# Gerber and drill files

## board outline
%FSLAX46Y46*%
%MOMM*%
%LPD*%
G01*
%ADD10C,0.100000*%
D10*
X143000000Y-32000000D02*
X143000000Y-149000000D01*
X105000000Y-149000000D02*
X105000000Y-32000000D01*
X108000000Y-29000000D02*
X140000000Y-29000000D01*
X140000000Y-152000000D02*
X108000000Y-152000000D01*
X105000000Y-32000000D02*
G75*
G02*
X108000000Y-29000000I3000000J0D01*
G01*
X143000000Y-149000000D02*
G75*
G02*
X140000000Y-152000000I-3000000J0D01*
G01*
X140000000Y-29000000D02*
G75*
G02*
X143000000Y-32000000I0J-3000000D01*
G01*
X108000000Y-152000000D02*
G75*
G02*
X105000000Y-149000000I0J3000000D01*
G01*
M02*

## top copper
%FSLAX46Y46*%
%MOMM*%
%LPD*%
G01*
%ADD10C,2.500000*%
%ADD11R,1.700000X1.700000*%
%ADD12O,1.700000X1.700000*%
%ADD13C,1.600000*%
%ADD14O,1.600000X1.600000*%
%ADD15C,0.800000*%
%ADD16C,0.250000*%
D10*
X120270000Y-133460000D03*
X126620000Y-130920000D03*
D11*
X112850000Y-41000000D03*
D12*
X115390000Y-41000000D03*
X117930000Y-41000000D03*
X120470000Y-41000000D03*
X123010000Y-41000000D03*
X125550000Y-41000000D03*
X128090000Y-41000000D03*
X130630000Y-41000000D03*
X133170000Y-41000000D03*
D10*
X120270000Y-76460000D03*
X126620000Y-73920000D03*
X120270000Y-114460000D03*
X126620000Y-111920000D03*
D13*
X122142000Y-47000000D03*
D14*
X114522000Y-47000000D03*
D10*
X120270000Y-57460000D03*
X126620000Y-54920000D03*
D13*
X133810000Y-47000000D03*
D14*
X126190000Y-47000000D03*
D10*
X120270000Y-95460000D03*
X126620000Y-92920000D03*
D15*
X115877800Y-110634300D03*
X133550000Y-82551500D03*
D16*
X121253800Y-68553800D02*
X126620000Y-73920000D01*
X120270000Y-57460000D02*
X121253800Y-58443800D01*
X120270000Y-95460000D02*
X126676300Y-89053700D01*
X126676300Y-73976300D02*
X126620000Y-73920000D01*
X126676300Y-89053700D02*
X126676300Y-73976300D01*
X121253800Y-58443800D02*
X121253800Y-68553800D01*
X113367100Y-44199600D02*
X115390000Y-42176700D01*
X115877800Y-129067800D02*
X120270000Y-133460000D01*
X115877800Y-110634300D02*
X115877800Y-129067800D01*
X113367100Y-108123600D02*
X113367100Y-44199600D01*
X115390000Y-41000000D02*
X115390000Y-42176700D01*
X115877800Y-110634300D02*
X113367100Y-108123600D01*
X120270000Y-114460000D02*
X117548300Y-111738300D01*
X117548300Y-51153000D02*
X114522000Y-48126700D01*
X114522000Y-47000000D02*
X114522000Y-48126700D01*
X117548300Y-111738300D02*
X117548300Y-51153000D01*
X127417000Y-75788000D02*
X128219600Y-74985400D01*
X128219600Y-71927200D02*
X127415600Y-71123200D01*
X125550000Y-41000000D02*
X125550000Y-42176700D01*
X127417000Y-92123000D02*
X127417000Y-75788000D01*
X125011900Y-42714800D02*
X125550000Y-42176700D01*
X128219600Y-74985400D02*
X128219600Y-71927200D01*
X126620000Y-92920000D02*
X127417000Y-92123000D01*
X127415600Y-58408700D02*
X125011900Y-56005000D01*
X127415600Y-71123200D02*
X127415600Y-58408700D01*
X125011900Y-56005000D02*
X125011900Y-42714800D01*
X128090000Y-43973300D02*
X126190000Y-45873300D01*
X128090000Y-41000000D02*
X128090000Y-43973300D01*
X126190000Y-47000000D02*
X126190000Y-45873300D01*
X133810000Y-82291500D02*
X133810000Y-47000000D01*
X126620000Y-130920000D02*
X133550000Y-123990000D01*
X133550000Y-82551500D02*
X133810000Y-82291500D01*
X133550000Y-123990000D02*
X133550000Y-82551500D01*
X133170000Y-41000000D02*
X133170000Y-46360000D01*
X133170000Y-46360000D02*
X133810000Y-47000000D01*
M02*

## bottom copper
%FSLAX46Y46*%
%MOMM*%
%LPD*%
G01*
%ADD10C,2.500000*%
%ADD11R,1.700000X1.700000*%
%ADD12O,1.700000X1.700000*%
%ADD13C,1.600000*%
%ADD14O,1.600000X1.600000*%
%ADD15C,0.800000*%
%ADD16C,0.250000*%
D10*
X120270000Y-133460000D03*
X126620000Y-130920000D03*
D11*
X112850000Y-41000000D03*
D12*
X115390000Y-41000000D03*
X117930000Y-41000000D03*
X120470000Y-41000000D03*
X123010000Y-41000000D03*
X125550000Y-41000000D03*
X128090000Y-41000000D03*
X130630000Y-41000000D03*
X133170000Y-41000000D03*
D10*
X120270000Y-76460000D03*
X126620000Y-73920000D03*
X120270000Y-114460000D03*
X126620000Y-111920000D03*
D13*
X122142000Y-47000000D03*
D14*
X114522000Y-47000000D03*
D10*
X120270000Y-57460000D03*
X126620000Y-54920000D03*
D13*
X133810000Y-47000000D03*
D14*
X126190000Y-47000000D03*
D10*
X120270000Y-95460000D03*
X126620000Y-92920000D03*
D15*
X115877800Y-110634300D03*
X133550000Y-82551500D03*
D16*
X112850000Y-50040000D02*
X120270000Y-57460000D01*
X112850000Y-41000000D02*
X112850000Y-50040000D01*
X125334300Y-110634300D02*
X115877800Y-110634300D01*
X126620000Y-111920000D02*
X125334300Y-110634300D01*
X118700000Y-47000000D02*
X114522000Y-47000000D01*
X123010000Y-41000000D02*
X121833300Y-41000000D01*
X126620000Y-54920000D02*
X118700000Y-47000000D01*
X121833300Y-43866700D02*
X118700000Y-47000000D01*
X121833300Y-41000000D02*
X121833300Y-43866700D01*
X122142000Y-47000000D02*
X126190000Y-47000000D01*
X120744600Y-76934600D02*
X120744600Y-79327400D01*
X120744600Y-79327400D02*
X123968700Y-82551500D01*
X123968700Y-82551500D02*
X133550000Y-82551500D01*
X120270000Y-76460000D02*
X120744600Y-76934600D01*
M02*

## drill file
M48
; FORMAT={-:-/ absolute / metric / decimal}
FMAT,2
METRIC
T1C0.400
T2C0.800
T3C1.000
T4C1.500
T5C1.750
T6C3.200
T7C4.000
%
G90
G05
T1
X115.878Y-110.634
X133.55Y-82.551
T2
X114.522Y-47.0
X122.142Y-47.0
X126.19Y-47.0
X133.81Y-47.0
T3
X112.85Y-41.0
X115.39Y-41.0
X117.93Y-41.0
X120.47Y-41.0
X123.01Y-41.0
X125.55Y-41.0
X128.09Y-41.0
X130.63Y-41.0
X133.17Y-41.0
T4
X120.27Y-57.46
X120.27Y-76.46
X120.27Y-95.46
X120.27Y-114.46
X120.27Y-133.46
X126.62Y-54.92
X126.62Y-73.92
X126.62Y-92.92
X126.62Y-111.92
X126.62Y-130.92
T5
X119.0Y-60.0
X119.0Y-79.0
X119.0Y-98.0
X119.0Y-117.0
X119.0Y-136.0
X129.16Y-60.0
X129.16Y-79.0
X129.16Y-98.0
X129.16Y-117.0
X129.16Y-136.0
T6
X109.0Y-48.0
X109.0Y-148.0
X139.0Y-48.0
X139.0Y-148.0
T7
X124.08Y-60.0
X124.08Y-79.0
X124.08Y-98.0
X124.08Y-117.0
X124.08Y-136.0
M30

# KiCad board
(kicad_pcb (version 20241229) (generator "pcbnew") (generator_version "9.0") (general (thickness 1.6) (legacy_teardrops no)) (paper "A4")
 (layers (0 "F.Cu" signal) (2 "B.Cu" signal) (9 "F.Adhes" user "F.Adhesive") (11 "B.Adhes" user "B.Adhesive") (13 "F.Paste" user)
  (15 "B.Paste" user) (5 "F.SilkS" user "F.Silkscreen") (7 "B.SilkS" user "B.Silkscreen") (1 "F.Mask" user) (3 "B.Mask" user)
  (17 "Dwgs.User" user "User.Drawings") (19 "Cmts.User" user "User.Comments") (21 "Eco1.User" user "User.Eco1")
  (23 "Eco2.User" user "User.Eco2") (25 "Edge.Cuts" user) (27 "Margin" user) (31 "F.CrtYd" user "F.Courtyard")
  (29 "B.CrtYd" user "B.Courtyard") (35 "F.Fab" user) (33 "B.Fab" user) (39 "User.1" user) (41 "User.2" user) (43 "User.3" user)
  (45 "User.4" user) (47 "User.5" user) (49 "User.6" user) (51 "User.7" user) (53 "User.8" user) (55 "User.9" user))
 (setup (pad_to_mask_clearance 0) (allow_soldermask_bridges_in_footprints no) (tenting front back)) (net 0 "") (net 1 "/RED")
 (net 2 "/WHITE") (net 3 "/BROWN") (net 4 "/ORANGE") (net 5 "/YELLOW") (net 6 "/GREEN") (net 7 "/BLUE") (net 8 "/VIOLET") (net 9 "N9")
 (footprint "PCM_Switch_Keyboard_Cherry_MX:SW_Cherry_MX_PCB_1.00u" (layer "F.Cu") (at 124.08 136)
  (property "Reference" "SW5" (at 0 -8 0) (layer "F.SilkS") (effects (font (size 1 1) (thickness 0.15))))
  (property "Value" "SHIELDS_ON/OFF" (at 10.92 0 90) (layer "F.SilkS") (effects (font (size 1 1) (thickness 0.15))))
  (pad "" np_thru_hole circle (at -5.08 0) (size 1.75 1.75) (drill 1.75) (layers "*.Cu" "*.Mask"))
  (pad "" np_thru_hole circle (at 0 0) (size 4 4) (drill 4) (layers "*.Cu" "*.Mask"))
  (pad "" np_thru_hole circle (at 5.08 0) (size 1.75 1.75) (drill 1.75) (layers "*.Cu" "*.Mask"))
  (pad "1" thru_hole circle (at -3.81 -2.54) (size 2.5 2.5) (drill 1.5) (layers "*.Cu" "*.Mask") (remove_unused_layers no) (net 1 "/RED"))
  (pad "2" thru_hole circle (at 2.54 -5.08) (size 2.5 2.5) (drill 1.5) (layers "*.Cu" "*.Mask") (remove_unused_layers no) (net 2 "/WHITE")))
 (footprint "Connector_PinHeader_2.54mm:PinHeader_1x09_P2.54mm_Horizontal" (layer "F.Cu") (at 112.85 41 90)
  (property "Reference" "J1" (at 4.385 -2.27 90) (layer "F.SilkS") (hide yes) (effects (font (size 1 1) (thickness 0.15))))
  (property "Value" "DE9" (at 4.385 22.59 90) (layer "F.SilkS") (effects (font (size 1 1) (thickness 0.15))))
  (pad "1" thru_hole rect (at 0 0 90) (size 1.7 1.7) (drill 1) (layers "*.Cu" "*.Mask") (remove_unused_layers no) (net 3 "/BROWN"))
  (pad "2" thru_hole oval (at 0 2.54 90) (size 1.7 1.7) (drill 1) (layers "*.Cu" "*.Mask") (remove_unused_layers no) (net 1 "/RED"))
  (pad "3" thru_hole oval (at 0 5.08 90) (size 1.7 1.7) (drill 1) (layers "*.Cu" "*.Mask") (remove_unused_layers no) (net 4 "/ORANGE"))
  (pad "4" thru_hole oval (at 0 7.62 90) (size 1.7 1.7) (drill 1) (layers "*.Cu" "*.Mask") (remove_unused_layers no) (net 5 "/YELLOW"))
  (pad "5" thru_hole oval (at 0 10.16 90) (size 1.7 1.7) (drill 1) (layers "*.Cu" "*.Mask") (remove_unused_layers no) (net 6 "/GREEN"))
  (pad "6" thru_hole oval (at 0 12.7 90) (size 1.7 1.7) (drill 1) (layers "*.Cu" "*.Mask") (remove_unused_layers no) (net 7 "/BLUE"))
  (pad "7" thru_hole oval (at 0 15.24 90) (size 1.7 1.7) (drill 1) (layers "*.Cu" "*.Mask") (remove_unused_layers no) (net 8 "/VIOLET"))
  (pad "8" thru_hole oval (at 0 17.78 90) (size 1.7 1.7) (drill 1) (layers "*.Cu" "*.Mask") (remove_unused_layers no) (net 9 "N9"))
  (pad "9" thru_hole oval (at 0 20.32 90) (size 1.7 1.7) (drill 1) (layers "*.Cu" "*.Mask") (remove_unused_layers no) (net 2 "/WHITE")))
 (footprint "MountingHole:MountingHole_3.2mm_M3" (layer "F.Cu") (at 109 48)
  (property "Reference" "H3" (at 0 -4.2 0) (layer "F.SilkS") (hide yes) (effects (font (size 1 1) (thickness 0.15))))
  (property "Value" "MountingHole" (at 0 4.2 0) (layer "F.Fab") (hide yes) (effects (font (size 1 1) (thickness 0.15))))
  (pad "" np_thru_hole circle (at 0 0) (size 3.2 3.2) (drill 3.2) (layers "*.Cu" "*.Mask")))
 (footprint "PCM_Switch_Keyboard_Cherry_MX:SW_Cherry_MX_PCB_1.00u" (layer "F.Cu") (at 124.08 79)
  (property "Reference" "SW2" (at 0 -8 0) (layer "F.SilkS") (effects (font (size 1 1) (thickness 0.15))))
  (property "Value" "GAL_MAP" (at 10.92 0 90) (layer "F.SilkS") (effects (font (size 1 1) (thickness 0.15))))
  (pad "" np_thru_hole circle (at -5.08 0) (size 1.75 1.75) (drill 1.75) (layers "*.Cu" "*.Mask"))
  (pad "" np_thru_hole circle (at 0 0) (size 4 4) (drill 4) (layers "*.Cu" "*.Mask"))
  (pad "" np_thru_hole circle (at 5.08 0) (size 1.75 1.75) (drill 1.75) (layers "*.Cu" "*.Mask"))
  (pad "1" thru_hole circle (at -3.81 -2.54) (size 2.5 2.5) (drill 1.5) (layers "*.Cu" "*.Mask") (remove_unused_layers no) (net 2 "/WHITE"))
  (pad "2" thru_hole circle (at 2.54 -5.08) (size 2.5 2.5) (drill 1.5) (layers "*.Cu" "*.Mask") (remove_unused_layers no) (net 3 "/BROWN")))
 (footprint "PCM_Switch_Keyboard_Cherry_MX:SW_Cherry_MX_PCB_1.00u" (layer "F.Cu") (at 124.08 117)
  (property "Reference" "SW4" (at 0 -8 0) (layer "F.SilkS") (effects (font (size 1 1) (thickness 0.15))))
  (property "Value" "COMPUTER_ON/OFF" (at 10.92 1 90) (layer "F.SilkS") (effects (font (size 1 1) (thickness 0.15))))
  (pad "" np_thru_hole circle (at -5.08 0) (size 1.75 1.75) (drill 1.75) (layers "*.Cu" "*.Mask"))
  (pad "" np_thru_hole circle (at 0 0) (size 4 4) (drill 4) (layers "*.Cu" "*.Mask"))
  (pad "" np_thru_hole circle (at 5.08 0) (size 1.75 1.75) (drill 1.75) (layers "*.Cu" "*.Mask"))
  (pad "1" thru_hole circle (at -3.81 -2.54) (size 2.5 2.5) (drill 1.5) (layers "*.Cu" "*.Mask") (remove_unused_layers no) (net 6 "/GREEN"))
  (pad "2" thru_hole circle (at 2.54 -5.08) (size 2.5 2.5) (drill 1.5) (layers "*.Cu" "*.Mask") (remove_unused_layers no) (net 1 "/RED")))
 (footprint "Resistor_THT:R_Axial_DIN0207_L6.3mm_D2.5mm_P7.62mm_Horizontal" (layer "F.Cu") (at 122.142 47 180)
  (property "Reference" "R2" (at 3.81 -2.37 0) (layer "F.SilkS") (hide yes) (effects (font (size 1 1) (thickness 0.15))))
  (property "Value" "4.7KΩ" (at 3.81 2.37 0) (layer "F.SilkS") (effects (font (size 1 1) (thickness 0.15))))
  (pad "1" thru_hole circle (at 0 0 180) (size 1.6 1.6) (drill 0.8) (layers "*.Cu" "*.Mask") (remove_unused_layers no) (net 8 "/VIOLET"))
  (pad "2" thru_hole oval (at 7.62 0 180) (size 1.6 1.6) (drill 0.8) (layers "*.Cu" "*.Mask") (remove_unused_layers no) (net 6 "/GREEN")))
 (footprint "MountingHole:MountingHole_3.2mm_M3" (layer "F.Cu") (at 139 148)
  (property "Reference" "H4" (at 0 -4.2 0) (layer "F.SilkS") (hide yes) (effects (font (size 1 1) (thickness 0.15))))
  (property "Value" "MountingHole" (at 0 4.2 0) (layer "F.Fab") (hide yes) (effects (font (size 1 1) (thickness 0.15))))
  (pad "" np_thru_hole circle (at 0 0) (size 3.2 3.2) (drill 3.2) (layers "*.Cu" "*.Mask")))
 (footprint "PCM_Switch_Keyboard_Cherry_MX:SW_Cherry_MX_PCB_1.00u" (layer "F.Cu") (at 124.08 60)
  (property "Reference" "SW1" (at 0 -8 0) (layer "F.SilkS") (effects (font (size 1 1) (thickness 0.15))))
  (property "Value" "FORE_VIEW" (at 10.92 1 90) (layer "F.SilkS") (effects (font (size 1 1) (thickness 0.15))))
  (pad "" np_thru_hole circle (at -5.08 0) (size 1.75 1.75) (drill 1.75) (layers "*.Cu" "*.Mask"))
  (pad "" np_thru_hole circle (at 0 0) (size 4 4) (drill 4) (layers "*.Cu" "*.Mask"))
  (pad "" np_thru_hole circle (at 5.08 0) (size 1.75 1.75) (drill 1.75) (layers "*.Cu" "*.Mask"))
  (pad "1" thru_hole circle (at -3.81 -2.54) (size 2.5 2.5) (drill 1.5) (layers "*.Cu" "*.Mask") (remove_unused_layers no) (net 3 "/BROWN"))
  (pad "2" thru_hole circle (at 2.54 -5.08) (size 2.5 2.5) (drill 1.5) (layers "*.Cu" "*.Mask") (remove_unused_layers no) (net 6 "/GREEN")))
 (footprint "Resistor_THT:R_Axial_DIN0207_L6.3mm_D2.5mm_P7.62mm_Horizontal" (layer "F.Cu") (at 133.81 47 180)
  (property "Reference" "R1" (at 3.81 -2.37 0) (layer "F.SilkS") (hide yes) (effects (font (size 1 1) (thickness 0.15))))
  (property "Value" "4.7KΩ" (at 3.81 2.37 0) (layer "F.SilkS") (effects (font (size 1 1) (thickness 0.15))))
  (pad "1" thru_hole circle (at 0 0 180) (size 1.6 1.6) (drill 0.8) (layers "*.Cu" "*.Mask") (remove_unused_layers no) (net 2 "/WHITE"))
  (pad "2" thru_hole oval (at 7.62 0 180) (size 1.6 1.6) (drill 0.8) (layers "*.Cu" "*.Mask") (remove_unused_layers no) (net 8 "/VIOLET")))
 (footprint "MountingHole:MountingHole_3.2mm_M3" (layer "F.Cu") (at 139 48)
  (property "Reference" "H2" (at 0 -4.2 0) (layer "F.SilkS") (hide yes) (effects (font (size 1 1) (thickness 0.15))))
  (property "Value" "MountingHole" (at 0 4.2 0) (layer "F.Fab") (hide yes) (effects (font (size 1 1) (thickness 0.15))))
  (pad "" np_thru_hole circle (at 0 0) (size 3.2 3.2) (drill 3.2) (layers "*.Cu" "*.Mask")))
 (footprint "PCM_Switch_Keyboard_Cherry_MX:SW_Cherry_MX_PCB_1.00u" (layer "F.Cu") (at 124.08 98)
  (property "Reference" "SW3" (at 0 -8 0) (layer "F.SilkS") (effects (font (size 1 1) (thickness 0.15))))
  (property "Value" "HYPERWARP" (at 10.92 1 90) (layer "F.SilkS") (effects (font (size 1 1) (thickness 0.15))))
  (pad "" np_thru_hole circle (at -5.08 0) (size 1.75 1.75) (drill 1.75) (layers "*.Cu" "*.Mask"))
  (pad "" np_thru_hole circle (at 0 0) (size 4 4) (drill 4) (layers "*.Cu" "*.Mask"))
  (pad "" np_thru_hole circle (at 5.08 0) (size 1.75 1.75) (drill 1.75) (layers "*.Cu" "*.Mask"))
  (pad "1" thru_hole circle (at -3.81 -2.54) (size 2.5 2.5) (drill 1.5) (layers "*.Cu" "*.Mask") (remove_unused_layers no) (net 3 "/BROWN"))
  (pad "2" thru_hole circle (at 2.54 -5.08) (size 2.5 2.5) (drill 1.5) (layers "*.Cu" "*.Mask") (remove_unused_layers no) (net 7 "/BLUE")))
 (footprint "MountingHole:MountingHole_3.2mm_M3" (layer "F.Cu") (at 109 148)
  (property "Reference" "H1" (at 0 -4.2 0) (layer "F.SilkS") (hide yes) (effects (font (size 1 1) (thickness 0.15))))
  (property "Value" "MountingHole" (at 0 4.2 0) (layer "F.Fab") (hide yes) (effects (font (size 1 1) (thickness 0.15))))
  (pad "" np_thru_hole circle (at 0 0) (size 3.2 3.2) (drill 3.2) (layers "*.Cu" "*.Mask")))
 (gr_line (start 143 32) (end 143 149) (stroke (width 0.1) (type default)) (layer "Edge.Cuts"))
 (gr_line (start 105 149) (end 105 32) (stroke (width 0.1) (type default)) (layer "Edge.Cuts"))
 (gr_line (start 108 29) (end 140 29) (stroke (width 0.1) (type default)) (layer "Edge.Cuts"))
 (gr_line (start 140 152) (end 108 152) (stroke (width 0.1) (type default)) (layer "Edge.Cuts"))
 (gr_arc (start 105 32) (mid 105.87868 29.87868) (end 108 29) (stroke (width 0.1) (type default)) (layer "Edge.Cuts"))
 (gr_arc (start 143 149) (mid 142.12132 151.12132) (end 140 152) (stroke (width 0.1) (type default)) (layer "Edge.Cuts"))
 (gr_arc (start 140 29) (mid 142.12132 29.87868) (end 143 32) (stroke (width 0.1) (type default)) (layer "Edge.Cuts"))
 (gr_arc (start 108 152) (mid 105.87868 151.12132) (end 105 149) (stroke (width 0.1) (type default)) (layer "Edge.Cuts"))
 (segment (start 121.2538 68.5538) (end 126.62 73.92) (width 0.25) (layer "F.Cu") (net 3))
 (segment (start 120.27 57.46) (end 121.2538 58.4438) (width 0.25) (layer "F.Cu") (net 3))
 (segment (start 120.27 95.46) (end 126.6763 89.0537) (width 0.25) (layer "F.Cu") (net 3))
 (segment (start 126.6763 73.9763) (end 126.62 73.92) (width 0.25) (layer "F.Cu") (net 3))
 (segment (start 126.6763 89.0537) (end 126.6763 73.9763) (width 0.25) (layer "F.Cu") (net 3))
 (segment (start 121.2538 58.4438) (end 121.2538 68.5538) (width 0.25) (layer "F.Cu") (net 3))
 (segment (start 112.85 50.04) (end 120.27 57.46) (width 0.25) (layer "B.Cu") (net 3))
 (segment (start 112.85 41) (end 112.85 50.04) (width 0.25) (layer "B.Cu") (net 3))
 (segment (start 113.3671 44.1996) (end 115.39 42.1767) (width 0.25) (layer "F.Cu") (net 1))
 (segment (start 115.8778 129.0678) (end 120.27 133.46) (width 0.25) (layer "F.Cu") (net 1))
 (segment (start 115.8778 110.6343) (end 115.8778 129.0678) (width 0.25) (layer "F.Cu") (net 1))
 (segment (start 113.3671 108.1236) (end 113.3671 44.1996) (width 0.25) (layer "F.Cu") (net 1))
 (segment (start 115.39 41) (end 115.39 42.1767) (width 0.25) (layer "F.Cu") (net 1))
 (segment (start 115.8778 110.6343) (end 113.3671 108.1236) (width 0.25) (layer "F.Cu") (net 1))
 (via (at 115.8778 110.6343) (size 0.8) (drill 0.4) (layers "F.Cu" "B.Cu") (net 1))
 (segment (start 125.3343 110.6343) (end 115.8778 110.6343) (width 0.25) (layer "B.Cu") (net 1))
 (segment (start 126.62 111.92) (end 125.3343 110.6343) (width 0.25) (layer "B.Cu") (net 1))
 (segment (start 120.27 114.46) (end 117.5483 111.7383) (width 0.25) (layer "F.Cu") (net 6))
 (segment (start 117.5483 51.153) (end 114.522 48.1267) (width 0.25) (layer "F.Cu") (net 6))
 (segment (start 114.522 47) (end 114.522 48.1267) (width 0.25) (layer "F.Cu") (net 6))
 (segment (start 117.5483 111.7383) (end 117.5483 51.153) (width 0.25) (layer "F.Cu") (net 6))
 (segment (start 118.7 47) (end 114.522 47) (width 0.25) (layer "B.Cu") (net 6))
 (segment (start 123.01 41) (end 121.8333 41) (width 0.25) (layer "B.Cu") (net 6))
 (segment (start 126.62 54.92) (end 118.7 47) (width 0.25) (layer "B.Cu") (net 6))
 (segment (start 121.8333 43.8667) (end 118.7 47) (width 0.25) (layer "B.Cu") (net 6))
 (segment (start 121.8333 41) (end 121.8333 43.8667) (width 0.25) (layer "B.Cu") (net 6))
 (segment (start 127.417 75.788) (end 128.2196 74.9854) (width 0.25) (layer "F.Cu") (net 7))
 (segment (start 128.2196 71.9272) (end 127.4156 71.1232) (width 0.25) (layer "F.Cu") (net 7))
 (segment (start 125.55 41) (end 125.55 42.1767) (width 0.25) (layer "F.Cu") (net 7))
 (segment (start 127.417 92.123) (end 127.417 75.788) (width 0.25) (layer "F.Cu") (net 7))
 (segment (start 125.0119 42.7148) (end 125.55 42.1767) (width 0.25) (layer "F.Cu") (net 7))
 (segment (start 128.2196 74.9854) (end 128.2196 71.9272) (width 0.25) (layer "F.Cu") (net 7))
 (segment (start 126.62 92.92) (end 127.417 92.123) (width 0.25) (layer "F.Cu") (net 7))
 (segment (start 127.4156 58.4087) (end 125.0119 56.005) (width 0.25) (layer "F.Cu") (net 7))
 (segment (start 127.4156 71.1232) (end 127.4156 58.4087) (width 0.25) (layer "F.Cu") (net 7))
 (segment (start 125.0119 56.005) (end 125.0119 42.7148) (width 0.25) (layer "F.Cu") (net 7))
 (segment (start 128.09 43.9733) (end 126.19 45.8733) (width 0.25) (layer "F.Cu") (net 8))
 (segment (start 128.09 41) (end 128.09 43.9733) (width 0.25) (layer "F.Cu") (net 8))
 (segment (start 126.19 47) (end 126.19 45.8733) (width 0.25) (layer "F.Cu") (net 8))
 (segment (start 122.142 47) (end 126.19 47) (width 0.25) (layer "B.Cu") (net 8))
 (segment (start 133.81 82.2915) (end 133.81 47) (width 0.25) (layer "F.Cu") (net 2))
 (segment (start 126.62 130.92) (end 133.55 123.99) (width 0.25) (layer "F.Cu") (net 2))
 (segment (start 133.55 82.5515) (end 133.81 82.2915) (width 0.25) (layer "F.Cu") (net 2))
 (segment (start 133.55 123.99) (end 133.55 82.5515) (width 0.25) (layer "F.Cu") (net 2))
 (segment (start 133.17 41) (end 133.17 46.36) (width 0.25) (layer "F.Cu") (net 2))
 (segment (start 133.17 46.36) (end 133.81 47) (width 0.25) (layer "F.Cu") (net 2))
 (via (at 133.55 82.5515) (size 0.8) (drill 0.4) (layers "F.Cu" "B.Cu") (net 2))
 (segment (start 120.7446 76.9346) (end 120.7446 79.3274) (width 0.25) (layer "B.Cu") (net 2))
 (segment (start 120.7446 79.3274) (end 123.9687 82.5515) (width 0.25) (layer "B.Cu") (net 2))
 (segment (start 123.9687 82.5515) (end 133.55 82.5515) (width 0.25) (layer "B.Cu") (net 2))
 (segment (start 120.27 76.46) (end 120.7446 76.9346) (width 0.25) (layer "B.Cu") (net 2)))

